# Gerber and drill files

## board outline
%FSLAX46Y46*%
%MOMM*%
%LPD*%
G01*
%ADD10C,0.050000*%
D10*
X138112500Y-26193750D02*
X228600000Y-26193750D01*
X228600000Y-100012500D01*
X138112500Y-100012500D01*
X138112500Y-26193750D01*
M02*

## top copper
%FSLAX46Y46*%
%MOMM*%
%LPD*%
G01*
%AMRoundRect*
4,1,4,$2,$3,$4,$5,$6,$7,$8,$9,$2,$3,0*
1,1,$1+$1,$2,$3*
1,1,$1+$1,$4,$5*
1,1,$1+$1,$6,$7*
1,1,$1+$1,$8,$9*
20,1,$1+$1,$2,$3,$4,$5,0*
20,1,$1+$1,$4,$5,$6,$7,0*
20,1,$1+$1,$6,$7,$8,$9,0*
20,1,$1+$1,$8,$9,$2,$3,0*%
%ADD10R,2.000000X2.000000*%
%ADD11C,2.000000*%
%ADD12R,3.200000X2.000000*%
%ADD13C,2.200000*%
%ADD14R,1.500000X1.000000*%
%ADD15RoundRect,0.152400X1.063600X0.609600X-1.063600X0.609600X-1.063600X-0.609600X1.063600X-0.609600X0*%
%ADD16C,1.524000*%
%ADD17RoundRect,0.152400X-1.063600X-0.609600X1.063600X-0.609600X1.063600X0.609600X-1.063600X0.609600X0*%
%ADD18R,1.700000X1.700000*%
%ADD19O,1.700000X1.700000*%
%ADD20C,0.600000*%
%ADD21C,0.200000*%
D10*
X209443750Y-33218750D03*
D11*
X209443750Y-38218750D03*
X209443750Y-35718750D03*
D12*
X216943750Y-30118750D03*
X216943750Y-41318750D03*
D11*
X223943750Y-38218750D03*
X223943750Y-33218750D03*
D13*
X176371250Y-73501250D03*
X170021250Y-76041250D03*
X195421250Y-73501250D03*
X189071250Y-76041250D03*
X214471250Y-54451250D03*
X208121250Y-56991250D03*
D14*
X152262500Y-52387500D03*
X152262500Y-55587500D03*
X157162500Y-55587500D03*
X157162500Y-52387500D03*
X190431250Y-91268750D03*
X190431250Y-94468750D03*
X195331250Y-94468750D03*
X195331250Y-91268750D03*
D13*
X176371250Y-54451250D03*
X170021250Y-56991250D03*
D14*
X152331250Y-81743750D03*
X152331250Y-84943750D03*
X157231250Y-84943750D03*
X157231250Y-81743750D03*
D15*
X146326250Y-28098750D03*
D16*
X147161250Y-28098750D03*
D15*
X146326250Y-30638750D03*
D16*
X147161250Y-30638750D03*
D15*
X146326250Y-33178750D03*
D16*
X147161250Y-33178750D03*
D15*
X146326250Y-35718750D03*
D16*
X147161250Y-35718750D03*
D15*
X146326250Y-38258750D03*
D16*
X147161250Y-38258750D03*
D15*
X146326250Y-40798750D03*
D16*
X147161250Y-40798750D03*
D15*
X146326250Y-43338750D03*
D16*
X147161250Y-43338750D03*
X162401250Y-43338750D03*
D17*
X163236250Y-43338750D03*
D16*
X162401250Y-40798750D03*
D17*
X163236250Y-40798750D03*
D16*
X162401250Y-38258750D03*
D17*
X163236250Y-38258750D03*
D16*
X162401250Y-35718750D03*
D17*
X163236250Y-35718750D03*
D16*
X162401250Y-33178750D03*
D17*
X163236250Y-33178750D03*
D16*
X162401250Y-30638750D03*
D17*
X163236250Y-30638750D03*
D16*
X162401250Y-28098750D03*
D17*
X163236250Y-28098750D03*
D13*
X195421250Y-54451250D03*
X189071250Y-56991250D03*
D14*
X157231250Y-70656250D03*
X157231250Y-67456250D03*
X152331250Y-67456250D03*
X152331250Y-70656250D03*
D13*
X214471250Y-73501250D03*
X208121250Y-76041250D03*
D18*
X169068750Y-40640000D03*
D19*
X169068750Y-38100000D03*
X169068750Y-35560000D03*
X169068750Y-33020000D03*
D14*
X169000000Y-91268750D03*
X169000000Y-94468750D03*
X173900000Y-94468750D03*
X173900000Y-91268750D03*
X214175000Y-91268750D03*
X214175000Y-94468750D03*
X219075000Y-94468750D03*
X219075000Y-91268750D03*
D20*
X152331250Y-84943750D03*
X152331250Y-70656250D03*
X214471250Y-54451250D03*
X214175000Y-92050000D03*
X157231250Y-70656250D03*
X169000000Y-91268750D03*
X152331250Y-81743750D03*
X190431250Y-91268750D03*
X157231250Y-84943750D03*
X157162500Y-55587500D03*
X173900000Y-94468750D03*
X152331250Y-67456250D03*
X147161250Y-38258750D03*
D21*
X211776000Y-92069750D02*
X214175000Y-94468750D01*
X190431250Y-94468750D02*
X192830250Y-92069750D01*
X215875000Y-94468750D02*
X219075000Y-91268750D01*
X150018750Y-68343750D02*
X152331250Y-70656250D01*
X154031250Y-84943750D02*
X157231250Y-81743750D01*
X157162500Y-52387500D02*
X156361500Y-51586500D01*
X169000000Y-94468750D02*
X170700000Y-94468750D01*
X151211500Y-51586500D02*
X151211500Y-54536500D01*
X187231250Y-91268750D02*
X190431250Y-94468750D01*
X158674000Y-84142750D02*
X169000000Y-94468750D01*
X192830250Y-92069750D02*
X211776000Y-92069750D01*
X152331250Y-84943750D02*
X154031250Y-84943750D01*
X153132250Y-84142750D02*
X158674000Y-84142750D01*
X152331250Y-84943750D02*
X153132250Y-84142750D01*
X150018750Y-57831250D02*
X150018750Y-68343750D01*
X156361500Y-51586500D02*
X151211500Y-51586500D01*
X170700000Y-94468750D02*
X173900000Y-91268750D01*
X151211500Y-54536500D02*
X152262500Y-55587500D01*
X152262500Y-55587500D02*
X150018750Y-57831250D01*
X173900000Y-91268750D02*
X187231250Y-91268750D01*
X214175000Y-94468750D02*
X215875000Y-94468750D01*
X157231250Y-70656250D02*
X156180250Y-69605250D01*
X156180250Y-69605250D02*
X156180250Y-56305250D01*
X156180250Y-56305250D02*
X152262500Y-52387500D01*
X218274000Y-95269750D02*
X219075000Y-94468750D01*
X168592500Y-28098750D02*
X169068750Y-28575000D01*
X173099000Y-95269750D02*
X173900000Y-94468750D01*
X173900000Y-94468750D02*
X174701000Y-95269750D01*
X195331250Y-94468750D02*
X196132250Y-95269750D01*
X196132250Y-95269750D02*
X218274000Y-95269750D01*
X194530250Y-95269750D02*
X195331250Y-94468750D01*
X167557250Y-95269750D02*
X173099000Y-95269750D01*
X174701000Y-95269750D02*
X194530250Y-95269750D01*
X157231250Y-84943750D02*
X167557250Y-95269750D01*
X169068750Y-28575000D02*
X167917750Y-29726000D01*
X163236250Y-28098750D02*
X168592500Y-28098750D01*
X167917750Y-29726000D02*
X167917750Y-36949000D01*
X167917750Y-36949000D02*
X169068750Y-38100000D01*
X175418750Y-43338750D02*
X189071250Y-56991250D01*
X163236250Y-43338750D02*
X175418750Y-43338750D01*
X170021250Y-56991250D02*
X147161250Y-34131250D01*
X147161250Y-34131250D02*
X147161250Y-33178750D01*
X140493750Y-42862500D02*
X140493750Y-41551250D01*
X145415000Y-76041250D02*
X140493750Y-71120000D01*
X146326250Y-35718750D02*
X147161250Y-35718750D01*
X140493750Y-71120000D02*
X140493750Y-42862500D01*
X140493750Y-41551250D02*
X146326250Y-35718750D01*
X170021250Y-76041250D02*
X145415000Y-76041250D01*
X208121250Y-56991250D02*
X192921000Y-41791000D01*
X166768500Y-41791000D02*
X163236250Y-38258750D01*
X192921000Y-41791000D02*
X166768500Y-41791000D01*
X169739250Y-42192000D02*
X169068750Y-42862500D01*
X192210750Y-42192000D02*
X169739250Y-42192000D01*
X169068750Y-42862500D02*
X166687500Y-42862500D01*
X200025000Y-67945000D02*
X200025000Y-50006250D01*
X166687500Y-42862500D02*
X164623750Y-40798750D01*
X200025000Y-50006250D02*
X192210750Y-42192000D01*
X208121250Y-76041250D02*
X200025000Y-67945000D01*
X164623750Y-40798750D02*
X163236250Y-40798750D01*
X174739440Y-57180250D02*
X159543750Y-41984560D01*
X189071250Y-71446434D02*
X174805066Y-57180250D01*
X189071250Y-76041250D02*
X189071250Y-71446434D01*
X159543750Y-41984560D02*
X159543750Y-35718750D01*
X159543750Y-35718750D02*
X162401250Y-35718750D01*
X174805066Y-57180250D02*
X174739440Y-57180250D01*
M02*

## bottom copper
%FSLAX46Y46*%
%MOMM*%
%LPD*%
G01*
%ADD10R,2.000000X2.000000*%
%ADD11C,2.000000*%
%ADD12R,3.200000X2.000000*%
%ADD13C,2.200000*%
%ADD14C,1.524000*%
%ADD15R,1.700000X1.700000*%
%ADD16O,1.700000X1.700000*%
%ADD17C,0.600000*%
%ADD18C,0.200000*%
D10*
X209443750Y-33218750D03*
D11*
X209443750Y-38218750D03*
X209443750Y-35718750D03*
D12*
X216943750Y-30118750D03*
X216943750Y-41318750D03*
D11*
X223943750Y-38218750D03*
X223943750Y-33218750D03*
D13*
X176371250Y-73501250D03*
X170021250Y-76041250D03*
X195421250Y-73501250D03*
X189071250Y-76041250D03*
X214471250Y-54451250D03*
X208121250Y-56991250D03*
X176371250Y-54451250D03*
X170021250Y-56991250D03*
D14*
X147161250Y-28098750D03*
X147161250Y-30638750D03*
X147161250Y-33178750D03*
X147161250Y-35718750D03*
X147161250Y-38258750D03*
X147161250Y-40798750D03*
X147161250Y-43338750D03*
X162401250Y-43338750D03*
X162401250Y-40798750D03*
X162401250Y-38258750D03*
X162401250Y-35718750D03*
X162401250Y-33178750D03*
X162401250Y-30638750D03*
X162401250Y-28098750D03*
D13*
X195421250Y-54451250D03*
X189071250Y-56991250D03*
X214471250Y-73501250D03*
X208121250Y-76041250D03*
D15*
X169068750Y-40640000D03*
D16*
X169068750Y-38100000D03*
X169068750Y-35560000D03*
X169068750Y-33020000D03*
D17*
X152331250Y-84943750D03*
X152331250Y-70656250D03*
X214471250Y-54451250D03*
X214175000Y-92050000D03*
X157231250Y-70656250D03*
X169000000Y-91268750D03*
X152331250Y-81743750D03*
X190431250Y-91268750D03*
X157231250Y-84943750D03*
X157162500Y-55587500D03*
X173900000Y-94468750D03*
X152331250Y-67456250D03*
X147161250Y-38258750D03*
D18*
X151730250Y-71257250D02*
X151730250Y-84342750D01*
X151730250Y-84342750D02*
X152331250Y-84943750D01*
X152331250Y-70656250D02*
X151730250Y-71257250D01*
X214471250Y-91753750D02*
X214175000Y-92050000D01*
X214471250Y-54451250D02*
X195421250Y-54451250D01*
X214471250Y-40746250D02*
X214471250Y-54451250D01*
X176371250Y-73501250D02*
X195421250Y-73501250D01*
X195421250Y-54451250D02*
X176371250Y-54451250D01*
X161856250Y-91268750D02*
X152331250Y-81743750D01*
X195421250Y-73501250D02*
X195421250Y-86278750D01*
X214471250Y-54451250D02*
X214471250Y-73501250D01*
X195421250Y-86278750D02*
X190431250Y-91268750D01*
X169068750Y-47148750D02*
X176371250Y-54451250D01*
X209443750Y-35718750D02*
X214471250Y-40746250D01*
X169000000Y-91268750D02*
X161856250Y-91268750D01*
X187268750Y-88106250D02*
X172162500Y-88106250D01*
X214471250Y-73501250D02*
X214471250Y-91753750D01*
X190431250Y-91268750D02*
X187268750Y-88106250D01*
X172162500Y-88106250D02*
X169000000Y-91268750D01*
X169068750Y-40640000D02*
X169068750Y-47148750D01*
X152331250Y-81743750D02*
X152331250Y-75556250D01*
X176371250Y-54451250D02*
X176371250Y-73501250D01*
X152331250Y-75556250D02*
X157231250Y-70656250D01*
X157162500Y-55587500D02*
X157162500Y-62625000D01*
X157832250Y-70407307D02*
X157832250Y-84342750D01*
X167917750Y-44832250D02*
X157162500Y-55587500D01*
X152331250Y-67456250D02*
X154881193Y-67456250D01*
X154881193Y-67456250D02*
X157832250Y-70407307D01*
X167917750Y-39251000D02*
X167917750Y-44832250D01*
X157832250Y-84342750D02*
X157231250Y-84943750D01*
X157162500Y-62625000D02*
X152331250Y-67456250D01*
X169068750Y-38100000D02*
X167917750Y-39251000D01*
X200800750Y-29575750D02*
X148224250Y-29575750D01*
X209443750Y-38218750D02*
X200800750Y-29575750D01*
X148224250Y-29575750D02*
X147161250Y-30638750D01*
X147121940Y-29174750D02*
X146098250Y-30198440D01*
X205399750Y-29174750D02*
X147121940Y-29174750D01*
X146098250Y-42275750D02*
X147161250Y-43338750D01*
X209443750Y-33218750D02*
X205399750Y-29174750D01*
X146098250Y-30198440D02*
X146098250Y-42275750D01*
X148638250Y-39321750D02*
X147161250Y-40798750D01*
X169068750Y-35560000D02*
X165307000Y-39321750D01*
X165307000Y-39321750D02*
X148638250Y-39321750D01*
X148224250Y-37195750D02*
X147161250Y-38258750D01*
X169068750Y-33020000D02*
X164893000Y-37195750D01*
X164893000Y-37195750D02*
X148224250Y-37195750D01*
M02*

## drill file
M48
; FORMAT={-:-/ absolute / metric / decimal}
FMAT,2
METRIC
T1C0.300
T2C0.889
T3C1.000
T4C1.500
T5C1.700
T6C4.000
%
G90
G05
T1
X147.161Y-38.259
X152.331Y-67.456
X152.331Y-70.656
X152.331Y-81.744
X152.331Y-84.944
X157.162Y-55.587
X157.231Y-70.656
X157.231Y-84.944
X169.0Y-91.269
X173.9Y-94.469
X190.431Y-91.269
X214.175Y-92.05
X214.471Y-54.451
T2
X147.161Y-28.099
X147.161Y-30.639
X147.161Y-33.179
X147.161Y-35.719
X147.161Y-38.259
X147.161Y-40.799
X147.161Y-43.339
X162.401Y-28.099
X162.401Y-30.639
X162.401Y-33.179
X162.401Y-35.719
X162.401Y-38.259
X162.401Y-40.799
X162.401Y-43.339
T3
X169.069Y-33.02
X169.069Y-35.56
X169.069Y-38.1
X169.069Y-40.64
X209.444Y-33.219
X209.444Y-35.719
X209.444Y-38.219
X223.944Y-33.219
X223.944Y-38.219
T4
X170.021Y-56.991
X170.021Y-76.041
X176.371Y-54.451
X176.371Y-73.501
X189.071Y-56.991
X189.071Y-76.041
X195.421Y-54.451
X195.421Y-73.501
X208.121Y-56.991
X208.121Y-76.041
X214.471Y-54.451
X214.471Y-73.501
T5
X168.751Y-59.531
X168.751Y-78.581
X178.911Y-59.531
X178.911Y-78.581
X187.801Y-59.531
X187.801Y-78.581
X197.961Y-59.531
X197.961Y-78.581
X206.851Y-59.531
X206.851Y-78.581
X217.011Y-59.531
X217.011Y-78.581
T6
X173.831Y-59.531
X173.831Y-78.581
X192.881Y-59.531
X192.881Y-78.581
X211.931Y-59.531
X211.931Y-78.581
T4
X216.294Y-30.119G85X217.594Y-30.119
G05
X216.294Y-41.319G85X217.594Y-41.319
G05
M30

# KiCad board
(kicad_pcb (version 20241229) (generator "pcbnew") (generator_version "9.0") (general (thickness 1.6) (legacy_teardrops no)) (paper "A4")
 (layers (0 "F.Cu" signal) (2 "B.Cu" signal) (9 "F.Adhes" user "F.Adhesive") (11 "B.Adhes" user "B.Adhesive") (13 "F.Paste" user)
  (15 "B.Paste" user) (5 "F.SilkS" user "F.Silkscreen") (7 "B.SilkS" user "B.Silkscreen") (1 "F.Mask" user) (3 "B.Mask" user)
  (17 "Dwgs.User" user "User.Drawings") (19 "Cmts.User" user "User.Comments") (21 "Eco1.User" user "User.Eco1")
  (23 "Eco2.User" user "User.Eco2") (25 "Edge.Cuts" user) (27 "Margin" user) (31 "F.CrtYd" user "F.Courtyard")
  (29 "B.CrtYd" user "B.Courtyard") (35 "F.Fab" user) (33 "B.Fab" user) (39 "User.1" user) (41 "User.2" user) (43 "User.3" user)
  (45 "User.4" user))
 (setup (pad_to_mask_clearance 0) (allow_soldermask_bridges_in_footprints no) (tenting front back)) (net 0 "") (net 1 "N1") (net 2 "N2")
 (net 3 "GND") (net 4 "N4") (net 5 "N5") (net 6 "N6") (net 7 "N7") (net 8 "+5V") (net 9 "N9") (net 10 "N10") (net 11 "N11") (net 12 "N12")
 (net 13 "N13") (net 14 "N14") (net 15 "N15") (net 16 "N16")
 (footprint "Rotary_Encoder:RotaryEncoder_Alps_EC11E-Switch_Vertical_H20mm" (layer "F.Cu") (at 209.44375 33.21875)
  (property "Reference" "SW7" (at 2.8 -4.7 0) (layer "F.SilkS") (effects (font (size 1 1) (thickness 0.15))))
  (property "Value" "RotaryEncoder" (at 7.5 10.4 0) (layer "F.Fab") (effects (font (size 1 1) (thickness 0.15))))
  (pad "A" thru_hole rect (at 0 0) (size 2 2) (drill 1) (layers "*.Cu" "*.Mask") (remove_unused_layers no) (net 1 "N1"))
  (pad "B" thru_hole circle (at 0 5) (size 2 2) (drill 1) (layers "*.Cu" "*.Mask") (remove_unused_layers no) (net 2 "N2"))
  (pad "C" thru_hole circle (at 0 2.5) (size 2 2) (drill 1) (layers "*.Cu" "*.Mask") (remove_unused_layers no) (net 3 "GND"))
  (pad "MP" thru_hole rect (at 7.5 -3.1) (size 3.2 2) (drill oval 2.8 1.5) (layers "*.Cu" "*.Mask") (remove_unused_layers no))
  (pad "MP" thru_hole rect (at 7.5 8.1) (size 3.2 2) (drill oval 2.8 1.5) (layers "*.Cu" "*.Mask") (remove_unused_layers no))
  (pad "S1" thru_hole circle (at 14.5 5) (size 2 2) (drill 1) (layers "*.Cu" "*.Mask") (remove_unused_layers no))
  (pad "S2" thru_hole circle (at 14.5 0) (size 2 2) (drill 1) (layers "*.Cu" "*.Mask") (remove_unused_layers no)))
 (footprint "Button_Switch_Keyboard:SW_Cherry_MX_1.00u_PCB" (layer "F.Cu") (at 176.37125 73.50125)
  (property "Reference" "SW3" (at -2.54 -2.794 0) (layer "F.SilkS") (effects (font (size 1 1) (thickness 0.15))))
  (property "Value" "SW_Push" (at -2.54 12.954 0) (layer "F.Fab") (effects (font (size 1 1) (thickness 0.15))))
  (pad "" np_thru_hole circle (at -7.62 5.08) (size 1.7 1.7) (drill 1.7) (layers "*.Cu" "*.Mask"))
  (pad "" np_thru_hole circle (at -2.54 5.08) (size 4 4) (drill 4) (layers "*.Cu" "*.Mask"))
  (pad "" np_thru_hole circle (at 2.54 5.08) (size 1.7 1.7) (drill 1.7) (layers "*.Cu" "*.Mask"))
  (pad "1" thru_hole circle (at 0 0) (size 2.2 2.2) (drill 1.5) (layers "*.Cu" "*.Mask") (remove_unused_layers no) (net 3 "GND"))
  (pad "2" thru_hole circle (at -6.35 2.54) (size 2.2 2.2) (drill 1.5) (layers "*.Cu" "*.Mask") (remove_unused_layers no) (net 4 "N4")))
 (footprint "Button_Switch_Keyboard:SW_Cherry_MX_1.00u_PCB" (layer "F.Cu") (at 195.42125 73.50125)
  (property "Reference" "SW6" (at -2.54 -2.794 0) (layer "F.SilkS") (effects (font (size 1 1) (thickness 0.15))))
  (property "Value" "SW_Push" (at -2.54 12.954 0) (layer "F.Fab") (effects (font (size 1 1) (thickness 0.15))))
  (pad "" np_thru_hole circle (at -7.62 5.08) (size 1.7 1.7) (drill 1.7) (layers "*.Cu" "*.Mask"))
  (pad "" np_thru_hole circle (at -2.54 5.08) (size 4 4) (drill 4) (layers "*.Cu" "*.Mask"))
  (pad "" np_thru_hole circle (at 2.54 5.08) (size 1.7 1.7) (drill 1.7) (layers "*.Cu" "*.Mask"))
  (pad "1" thru_hole circle (at 0 0) (size 2.2 2.2) (drill 1.5) (layers "*.Cu" "*.Mask") (remove_unused_layers no) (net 3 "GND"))
  (pad "2" thru_hole circle (at -6.35 2.54) (size 2.2 2.2) (drill 1.5) (layers "*.Cu" "*.Mask") (remove_unused_layers no) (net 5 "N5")))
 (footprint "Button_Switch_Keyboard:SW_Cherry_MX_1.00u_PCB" (layer "F.Cu") (at 214.47125 54.45125)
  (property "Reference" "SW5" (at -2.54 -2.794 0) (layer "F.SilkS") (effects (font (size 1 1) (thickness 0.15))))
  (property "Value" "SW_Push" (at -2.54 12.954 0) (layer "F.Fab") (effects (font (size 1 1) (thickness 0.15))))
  (pad "" np_thru_hole circle (at -7.62 5.08) (size 1.7 1.7) (drill 1.7) (layers "*.Cu" "*.Mask"))
  (pad "" np_thru_hole circle (at -2.54 5.08) (size 4 4) (drill 4) (layers "*.Cu" "*.Mask"))
  (pad "" np_thru_hole circle (at 2.54 5.08) (size 1.7 1.7) (drill 1.7) (layers "*.Cu" "*.Mask"))
  (pad "1" thru_hole circle (at 0 0) (size 2.2 2.2) (drill 1.5) (layers "*.Cu" "*.Mask") (remove_unused_layers no) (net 3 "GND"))
  (pad "2" thru_hole circle (at -6.35 2.54) (size 2.2 2.2) (drill 1.5) (layers "*.Cu" "*.Mask") (remove_unused_layers no) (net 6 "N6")))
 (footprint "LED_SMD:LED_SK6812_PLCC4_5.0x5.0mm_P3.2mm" (layer "F.Cu") (at 154.7125 53.9875)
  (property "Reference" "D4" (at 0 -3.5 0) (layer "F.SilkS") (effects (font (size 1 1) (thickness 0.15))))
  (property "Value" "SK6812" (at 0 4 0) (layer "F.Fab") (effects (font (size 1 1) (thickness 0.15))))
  (pad "1" smd rect (at -2.45 -1.6 180) (size 1.5 1) (layers "F.Cu" "F.Mask" "F.Paste") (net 3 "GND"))
  (pad "2" smd rect (at -2.45 1.6 180) (size 1.5 1) (layers "F.Cu" "F.Mask" "F.Paste") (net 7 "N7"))
  (pad "3" smd rect (at 2.45 1.6 180) (size 1.5 1) (layers "F.Cu" "F.Mask" "F.Paste") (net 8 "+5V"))
  (pad "4" smd rect (at 2.45 -1.6 180) (size 1.5 1) (layers "F.Cu" "F.Mask" "F.Paste") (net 7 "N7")))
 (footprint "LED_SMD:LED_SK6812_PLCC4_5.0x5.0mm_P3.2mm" (layer "F.Cu") (at 192.88125 92.86875)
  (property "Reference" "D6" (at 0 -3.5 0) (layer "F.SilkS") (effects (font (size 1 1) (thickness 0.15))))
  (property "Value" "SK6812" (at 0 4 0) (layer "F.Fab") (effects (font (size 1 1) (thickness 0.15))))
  (pad "1" smd rect (at -2.45 -1.6 180) (size 1.5 1) (layers "F.Cu" "F.Mask" "F.Paste") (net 3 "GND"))
  (pad "2" smd rect (at -2.45 1.6 180) (size 1.5 1) (layers "F.Cu" "F.Mask" "F.Paste") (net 7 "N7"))
  (pad "3" smd rect (at 2.45 1.6 180) (size 1.5 1) (layers "F.Cu" "F.Mask" "F.Paste") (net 8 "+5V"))
  (pad "4" smd rect (at 2.45 -1.6 180) (size 1.5 1) (layers "F.Cu" "F.Mask" "F.Paste") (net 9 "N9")))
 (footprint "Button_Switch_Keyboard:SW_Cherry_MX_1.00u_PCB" (layer "F.Cu") (at 176.37125 54.45125)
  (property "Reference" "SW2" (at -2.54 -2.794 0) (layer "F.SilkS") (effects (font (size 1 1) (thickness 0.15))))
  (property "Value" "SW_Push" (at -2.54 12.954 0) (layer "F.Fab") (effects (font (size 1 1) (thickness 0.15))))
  (pad "" np_thru_hole circle (at -7.62 5.08) (size 1.7 1.7) (drill 1.7) (layers "*.Cu" "*.Mask"))
  (pad "" np_thru_hole circle (at -2.54 5.08) (size 4 4) (drill 4) (layers "*.Cu" "*.Mask"))
  (pad "" np_thru_hole circle (at 2.54 5.08) (size 1.7 1.7) (drill 1.7) (layers "*.Cu" "*.Mask"))
  (pad "1" thru_hole circle (at 0 0) (size 2.2 2.2) (drill 1.5) (layers "*.Cu" "*.Mask") (remove_unused_layers no) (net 3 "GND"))
  (pad "2" thru_hole circle (at -6.35 2.54) (size 2.2 2.2) (drill 1.5) (layers "*.Cu" "*.Mask") (remove_unused_layers no) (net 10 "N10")))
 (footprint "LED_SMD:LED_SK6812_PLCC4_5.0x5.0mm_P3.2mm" (layer "F.Cu") (at 154.78125 83.34375)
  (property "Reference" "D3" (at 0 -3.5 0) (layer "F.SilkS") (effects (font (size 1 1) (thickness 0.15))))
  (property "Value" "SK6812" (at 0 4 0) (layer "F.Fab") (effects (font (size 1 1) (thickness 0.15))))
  (pad "1" smd rect (at -2.45 -1.6 180) (size 1.5 1) (layers "F.Cu" "F.Mask" "F.Paste") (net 3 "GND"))
  (pad "2" smd rect (at -2.45 1.6 180) (size 1.5 1) (layers "F.Cu" "F.Mask" "F.Paste") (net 7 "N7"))
  (pad "3" smd rect (at 2.45 1.6 180) (size 1.5 1) (layers "F.Cu" "F.Mask" "F.Paste") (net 8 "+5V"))
  (pad "4" smd rect (at 2.45 -1.6 180) (size 1.5 1) (layers "F.Cu" "F.Mask" "F.Paste") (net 7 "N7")))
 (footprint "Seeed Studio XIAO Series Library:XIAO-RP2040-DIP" (layer "F.Cu") (at 154.78125 35.71875)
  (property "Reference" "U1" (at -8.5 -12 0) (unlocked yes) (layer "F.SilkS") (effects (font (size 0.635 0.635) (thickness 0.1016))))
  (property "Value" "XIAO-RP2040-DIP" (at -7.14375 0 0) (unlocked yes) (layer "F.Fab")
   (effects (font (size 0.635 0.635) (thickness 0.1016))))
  (pad "1" smd roundrect (at -8.455 -7.62 180) (size 2.432 1.524) (layers "F.Cu" "F.Mask") (roundrect_rratio 0.1) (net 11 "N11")
   (thermal_bridge_angle 45))
  (pad "1" thru_hole circle (at -7.62 -7.62 180) (size 1.524 1.524) (drill 0.889) (layers "*.Cu" "*.Mask") (remove_unused_layers no)
   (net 11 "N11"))
  (pad "2" smd roundrect (at -8.455 -5.08 180) (size 2.432 1.524) (layers "F.Cu" "F.Mask") (roundrect_rratio 0.1) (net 2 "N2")
   (thermal_bridge_angle 45))
  (pad "2" thru_hole circle (at -7.62 -5.08 180) (size 1.524 1.524) (drill 0.889) (layers "*.Cu" "*.Mask") (remove_unused_layers no)
   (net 2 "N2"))
  (pad "3" smd roundrect (at -8.455 -2.54 180) (size 2.432 1.524) (layers "F.Cu" "F.Mask") (roundrect_rratio 0.1) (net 10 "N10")
   (thermal_bridge_angle 45))
  (pad "3" thru_hole circle (at -7.62 -2.54 180) (size 1.524 1.524) (drill 0.889) (layers "*.Cu" "*.Mask") (remove_unused_layers no)
   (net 10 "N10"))
  (pad "4" smd roundrect (at -8.455 0 180) (size 2.432 1.524) (layers "F.Cu" "F.Mask") (roundrect_rratio 0.1) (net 4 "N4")
   (thermal_bridge_angle 45))
  (pad "4" thru_hole circle (at -7.62 0 180) (size 1.524 1.524) (drill 0.889) (layers "*.Cu" "*.Mask") (remove_unused_layers no)
   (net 4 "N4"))
  (pad "5" smd roundrect (at -8.455 2.54 180) (size 2.432 1.524) (layers "F.Cu" "F.Mask") (roundrect_rratio 0.1) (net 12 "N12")
   (thermal_bridge_angle 45))
  (pad "5" thru_hole circle (at -7.62 2.54 180) (size 1.524 1.524) (drill 0.889) (layers "*.Cu" "*.Mask") (remove_unused_layers no)
   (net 12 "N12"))
  (pad "6" smd roundrect (at -8.455 5.08 180) (size 2.432 1.524) (layers "F.Cu" "F.Mask") (roundrect_rratio 0.1) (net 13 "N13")
   (thermal_bridge_angle 45))
  (pad "6" thru_hole circle (at -7.62 5.08 180) (size 1.524 1.524) (drill 0.889) (layers "*.Cu" "*.Mask") (remove_unused_layers no)
   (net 13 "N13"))
  (pad "7" smd roundrect (at -8.455 7.62 180) (size 2.432 1.524) (layers "F.Cu" "F.Mask") (roundrect_rratio 0.1) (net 1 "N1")
   (thermal_bridge_angle 45))
  (pad "7" thru_hole circle (at -7.62 7.62 180) (size 1.524 1.524) (drill 0.889) (layers "*.Cu" "*.Mask") (remove_unused_layers no)
   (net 1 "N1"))
  (pad "8" thru_hole circle (at 7.62 7.62) (size 1.524 1.524) (drill 0.889) (layers "*.Cu" "*.Mask") (remove_unused_layers no)
   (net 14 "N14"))
  (pad "8" smd roundrect (at 8.455 7.62) (size 2.432 1.524) (layers "F.Cu" "F.Mask") (roundrect_rratio 0.1) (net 14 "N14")
   (thermal_bridge_angle 45))
  (pad "9" thru_hole circle (at 7.62 5.08) (size 1.524 1.524) (drill 0.889) (layers "*.Cu" "*.Mask") (remove_unused_layers no)
   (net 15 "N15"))
  (pad "9" smd roundrect (at 8.455 5.08) (size 2.432 1.524) (layers "F.Cu" "F.Mask") (roundrect_rratio 0.1) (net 15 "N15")
   (thermal_bridge_angle 45))
  (pad "10" thru_hole circle (at 7.62 2.54) (size 1.524 1.524) (drill 0.889) (layers "*.Cu" "*.Mask") (remove_unused_layers no) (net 6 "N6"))
  (pad "10" smd roundrect (at 8.455 2.54) (size 2.432 1.524) (layers "F.Cu" "F.Mask") (roundrect_rratio 0.1) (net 6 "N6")
   (thermal_bridge_angle 45))
  (pad "11" thru_hole circle (at 7.62 0) (size 1.524 1.524) (drill 0.889) (layers "*.Cu" "*.Mask") (remove_unused_layers no) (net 5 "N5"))
  (pad "11" smd roundrect (at 8.455 0) (size 2.432 1.524) (layers "F.Cu" "F.Mask") (roundrect_rratio 0.1) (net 5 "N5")
   (thermal_bridge_angle 45))
  (pad "12" thru_hole circle (at 7.62 -2.54) (size 1.524 1.524) (drill 0.889) (layers "*.Cu" "*.Mask") (remove_unused_layers no)
   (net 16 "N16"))
  (pad "12" smd roundrect (at 8.455 -2.54) (size 2.432 1.524) (layers "F.Cu" "F.Mask") (roundrect_rratio 0.1) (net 16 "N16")
   (thermal_bridge_angle 45))
  (pad "13" thru_hole circle (at 7.62 -5.08) (size 1.524 1.524) (drill 0.889) (layers "*.Cu" "*.Mask") (remove_unused_layers no)
   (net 3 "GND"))
  (pad "13" smd roundrect (at 8.455 -5.08) (size 2.432 1.524) (layers "F.Cu" "F.Mask") (roundrect_rratio 0.1) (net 3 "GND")
   (thermal_bridge_angle 45))
  (pad "14" thru_hole circle (at 7.62 -7.62) (size 1.524 1.524) (drill 0.889) (layers "*.Cu" "*.Mask") (remove_unused_layers no)
   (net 8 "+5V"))
  (pad "14" smd roundrect (at 8.455 -7.62) (size 2.432 1.524) (layers "F.Cu" "F.Mask") (roundrect_rratio 0.1) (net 8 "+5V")
   (thermal_bridge_angle 45)))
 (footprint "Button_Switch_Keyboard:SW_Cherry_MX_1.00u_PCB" (layer "F.Cu") (at 195.42125 54.45125)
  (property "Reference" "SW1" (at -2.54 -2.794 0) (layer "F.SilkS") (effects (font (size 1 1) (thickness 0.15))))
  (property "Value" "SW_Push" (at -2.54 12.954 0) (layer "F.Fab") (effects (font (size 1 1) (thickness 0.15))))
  (pad "" np_thru_hole circle (at -7.62 5.08) (size 1.7 1.7) (drill 1.7) (layers "*.Cu" "*.Mask"))
  (pad "" np_thru_hole circle (at -2.54 5.08) (size 4 4) (drill 4) (layers "*.Cu" "*.Mask"))
  (pad "" np_thru_hole circle (at 2.54 5.08) (size 1.7 1.7) (drill 1.7) (layers "*.Cu" "*.Mask"))
  (pad "1" thru_hole circle (at 0 0) (size 2.2 2.2) (drill 1.5) (layers "*.Cu" "*.Mask") (remove_unused_layers no) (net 3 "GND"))
  (pad "2" thru_hole circle (at -6.35 2.54) (size 2.2 2.2) (drill 1.5) (layers "*.Cu" "*.Mask") (remove_unused_layers no) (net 14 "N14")))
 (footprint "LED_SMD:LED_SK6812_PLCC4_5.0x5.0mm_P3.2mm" (layer "F.Cu") (at 154.78125 69.05625 180)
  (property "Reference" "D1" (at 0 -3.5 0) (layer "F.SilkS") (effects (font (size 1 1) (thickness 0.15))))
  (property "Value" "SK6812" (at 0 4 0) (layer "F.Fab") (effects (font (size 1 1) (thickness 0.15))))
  (pad "1" smd rect (at -2.45 -1.6) (size 1.5 1) (layers "F.Cu" "F.Mask" "F.Paste") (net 3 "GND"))
  (pad "2" smd rect (at -2.45 1.6) (size 1.5 1) (layers "F.Cu" "F.Mask" "F.Paste") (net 11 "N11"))
  (pad "3" smd rect (at 2.45 1.6) (size 1.5 1) (layers "F.Cu" "F.Mask" "F.Paste") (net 8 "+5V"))
  (pad "4" smd rect (at 2.45 -1.6) (size 1.5 1) (layers "F.Cu" "F.Mask" "F.Paste") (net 7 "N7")))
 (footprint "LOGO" (layer "F.Cu") (at 145.25625 57.15)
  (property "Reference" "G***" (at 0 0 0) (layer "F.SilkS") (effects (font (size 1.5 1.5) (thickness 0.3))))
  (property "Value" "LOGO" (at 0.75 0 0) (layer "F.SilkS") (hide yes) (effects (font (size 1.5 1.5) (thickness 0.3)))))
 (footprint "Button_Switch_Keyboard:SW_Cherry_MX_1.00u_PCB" (layer "F.Cu") (at 214.47125 73.50125)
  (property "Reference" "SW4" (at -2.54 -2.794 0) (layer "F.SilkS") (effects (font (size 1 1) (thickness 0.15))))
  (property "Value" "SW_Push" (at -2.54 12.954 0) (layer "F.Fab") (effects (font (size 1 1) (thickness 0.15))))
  (pad "" np_thru_hole circle (at -7.62 5.08) (size 1.7 1.7) (drill 1.7) (layers "*.Cu" "*.Mask"))
  (pad "" np_thru_hole circle (at -2.54 5.08) (size 4 4) (drill 4) (layers "*.Cu" "*.Mask"))
  (pad "" np_thru_hole circle (at 2.54 5.08) (size 1.7 1.7) (drill 1.7) (layers "*.Cu" "*.Mask"))
  (pad "1" thru_hole circle (at 0 0) (size 2.2 2.2) (drill 1.5) (layers "*.Cu" "*.Mask") (remove_unused_layers no) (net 3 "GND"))
  (pad "2" thru_hole circle (at -6.35 2.54) (size 2.2 2.2) (drill 1.5) (layers "*.Cu" "*.Mask") (remove_unused_layers no) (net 15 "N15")))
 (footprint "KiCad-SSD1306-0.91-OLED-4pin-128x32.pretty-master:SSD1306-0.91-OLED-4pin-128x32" (layer "F.Cu") (at 205.56875 42.83 180)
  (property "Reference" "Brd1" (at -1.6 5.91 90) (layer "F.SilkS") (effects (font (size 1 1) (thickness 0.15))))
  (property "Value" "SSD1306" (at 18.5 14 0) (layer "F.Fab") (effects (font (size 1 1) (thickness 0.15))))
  (pad "1" thru_hole rect (at 36.5 2.19 180) (size 1.7 1.7) (drill 1) (layers "*.Cu" "*.Mask") (remove_unused_layers no) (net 3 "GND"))
  (pad "2" thru_hole oval (at 36.5 4.73 180) (size 1.7 1.7) (drill 1) (layers "*.Cu" "*.Mask") (remove_unused_layers no) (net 8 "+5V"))
  (pad "3" thru_hole oval (at 36.5 7.27 180) (size 1.7 1.7) (drill 1) (layers "*.Cu" "*.Mask") (remove_unused_layers no) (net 13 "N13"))
  (pad "4" thru_hole oval (at 36.5 9.81 180) (size 1.7 1.7) (drill 1) (layers "*.Cu" "*.Mask") (remove_unused_layers no) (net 12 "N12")))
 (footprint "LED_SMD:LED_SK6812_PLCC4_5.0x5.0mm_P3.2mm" (layer "F.Cu") (at 171.45 92.86875)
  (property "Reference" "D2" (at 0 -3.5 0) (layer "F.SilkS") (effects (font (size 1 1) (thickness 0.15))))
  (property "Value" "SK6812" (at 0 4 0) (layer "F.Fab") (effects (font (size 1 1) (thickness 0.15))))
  (pad "1" smd rect (at -2.45 -1.6 180) (size 1.5 1) (layers "F.Cu" "F.Mask" "F.Paste") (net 3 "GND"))
  (pad "2" smd rect (at -2.45 1.6 180) (size 1.5 1) (layers "F.Cu" "F.Mask" "F.Paste") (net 7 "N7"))
  (pad "3" smd rect (at 2.45 1.6 180) (size 1.5 1) (layers "F.Cu" "F.Mask" "F.Paste") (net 8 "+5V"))
  (pad "4" smd rect (at 2.45 -1.6 180) (size 1.5 1) (layers "F.Cu" "F.Mask" "F.Paste") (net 7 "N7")))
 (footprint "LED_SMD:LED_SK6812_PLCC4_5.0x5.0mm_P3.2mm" (layer "F.Cu") (at 216.625 92.86875)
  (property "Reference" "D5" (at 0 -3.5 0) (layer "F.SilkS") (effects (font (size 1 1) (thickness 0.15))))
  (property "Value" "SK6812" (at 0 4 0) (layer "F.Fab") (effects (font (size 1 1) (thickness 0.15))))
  (pad "1" smd rect (at -2.45 -1.6 180) (size 1.5 1) (layers "F.Cu" "F.Mask" "F.Paste") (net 3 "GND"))
  (pad "2" smd rect (at -2.45 1.6 180) (size 1.5 1) (layers "F.Cu" "F.Mask" "F.Paste") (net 7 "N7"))
  (pad "3" smd rect (at 2.45 1.6 180) (size 1.5 1) (layers "F.Cu" "F.Mask" "F.Paste") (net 8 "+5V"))
  (pad "4" smd rect (at 2.45 -1.6 180) (size 1.5 1) (layers "F.Cu" "F.Mask" "F.Paste") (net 7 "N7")))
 (gr_rect (start 138.1125 26.19375) (end 228.6 100.0125) (stroke (width 0.05) (type default)) (fill no) (layer "Edge.Cuts"))
 (segment (start 211.776 92.06975) (end 214.175 94.46875) (width 0.2) (layer "F.Cu") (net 7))
 (segment (start 190.43125 94.46875) (end 192.83025 92.06975) (width 0.2) (layer "F.Cu") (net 7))
 (segment (start 215.875 94.46875) (end 219.075 91.26875) (width 0.2) (layer "F.Cu") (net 7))
 (segment (start 150.01875 68.34375) (end 152.33125 70.65625) (width 0.2) (layer "F.Cu") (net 7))
 (segment (start 154.03125 84.94375) (end 157.23125 81.74375) (width 0.2) (layer "F.Cu") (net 7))
 (segment (start 157.1625 52.3875) (end 156.3615 51.5865) (width 0.2) (layer "F.Cu") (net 7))
 (segment (start 169 94.46875) (end 170.7 94.46875) (width 0.2) (layer "F.Cu") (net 7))
 (segment (start 151.2115 51.5865) (end 151.2115 54.5365) (width 0.2) (layer "F.Cu") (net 7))
 (segment (start 187.23125 91.26875) (end 190.43125 94.46875) (width 0.2) (layer "F.Cu") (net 7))
 (segment (start 158.674 84.14275) (end 169 94.46875) (width 0.2) (layer "F.Cu") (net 7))
 (segment (start 192.83025 92.06975) (end 211.776 92.06975) (width 0.2) (layer "F.Cu") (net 7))
 (segment (start 152.33125 84.94375) (end 154.03125 84.94375) (width 0.2) (layer "F.Cu") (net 7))
 (segment (start 153.13225 84.14275) (end 158.674 84.14275) (width 0.2) (layer "F.Cu") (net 7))
 (segment (start 152.33125 84.94375) (end 153.13225 84.14275) (width 0.2) (layer "F.Cu") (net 7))
 (segment (start 150.01875 57.83125) (end 150.01875 68.34375) (width 0.2) (layer "F.Cu") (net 7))
 (segment (start 156.3615 51.5865) (end 151.2115 51.5865) (width 0.2) (layer "F.Cu") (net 7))
 (segment (start 170.7 94.46875) (end 173.9 91.26875) (width 0.2) (layer "F.Cu") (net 7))
 (segment (start 151.2115 54.5365) (end 152.2625 55.5875) (width 0.2) (layer "F.Cu") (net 7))
 (segment (start 152.2625 55.5875) (end 150.01875 57.83125) (width 0.2) (layer "F.Cu") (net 7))
 (segment (start 173.9 91.26875) (end 187.23125 91.26875) (width 0.2) (layer "F.Cu") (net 7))
 (segment (start 214.175 94.46875) (end 215.875 94.46875) (width 0.2) (layer "F.Cu") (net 7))
 (via (at 152.33125 84.94375) (size 0.6) (drill 0.3) (layers "F.Cu" "B.Cu") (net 7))
 (via (at 152.33125 70.65625) (size 0.6) (drill 0.3) (layers "F.Cu" "B.Cu") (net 7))
 (segment (start 151.73025 71.25725) (end 151.73025 84.34275) (width 0.2) (layer "B.Cu") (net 7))
 (segment (start 151.73025 84.34275) (end 152.33125 84.94375) (width 0.2) (layer "B.Cu") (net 7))
 (segment (start 152.33125 70.65625) (end 151.73025 71.25725) (width 0.2) (layer "B.Cu") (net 7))
 (segment (start 157.23125 70.65625) (end 156.18025 69.60525) (width 0.2) (layer "F.Cu") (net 3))
 (segment (start 156.18025 69.60525) (end 156.18025 56.30525) (width 0.2) (layer "F.Cu") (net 3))
 (segment (start 156.18025 56.30525) (end 152.2625 52.3875) (width 0.2) (layer "F.Cu") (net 3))
 (via (at 214.47125 54.45125) (size 0.6) (drill 0.3) (layers "F.Cu" "B.Cu") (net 3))
 (via (at 214.175 92.05) (size 0.6) (drill 0.3) (layers "F.Cu" "B.Cu") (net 3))
 (via (at 157.23125 70.65625) (size 0.6) (drill 0.3) (layers "F.Cu" "B.Cu") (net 3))
 (via (at 169 91.26875) (size 0.6) (drill 0.3) (layers "F.Cu" "B.Cu") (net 3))
 (via (at 152.33125 81.74375) (size 0.6) (drill 0.3) (layers "F.Cu" "B.Cu") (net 3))
 (via (at 190.43125 91.26875) (size 0.6) (drill 0.3) (layers "F.Cu" "B.Cu") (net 3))
 (segment (start 214.47125 91.75375) (end 214.175 92.05) (width 0.2) (layer "B.Cu") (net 3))
 (segment (start 214.47125 54.45125) (end 195.42125 54.45125) (width 0.2) (layer "B.Cu") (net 3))
 (segment (start 214.47125 40.74625) (end 214.47125 54.45125) (width 0.2) (layer "B.Cu") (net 3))
 (segment (start 176.37125 73.50125) (end 195.42125 73.50125) (width 0.2) (layer "B.Cu") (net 3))
 (segment (start 195.42125 54.45125) (end 176.37125 54.45125) (width 0.2) (layer "B.Cu") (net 3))
 (segment (start 161.85625 91.26875) (end 152.33125 81.74375) (width 0.2) (layer "B.Cu") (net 3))
 (segment (start 195.42125 73.50125) (end 195.42125 86.27875) (width 0.2) (layer "B.Cu") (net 3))
 (segment (start 214.47125 54.45125) (end 214.47125 73.50125) (width 0.2) (layer "B.Cu") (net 3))
 (segment (start 195.42125 86.27875) (end 190.43125 91.26875) (width 0.2) (layer "B.Cu") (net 3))
 (segment (start 169.06875 47.14875) (end 176.37125 54.45125) (width 0.2) (layer "B.Cu") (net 3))
 (segment (start 209.44375 35.71875) (end 214.47125 40.74625) (width 0.2) (layer "B.Cu") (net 3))
 (segment (start 169 91.26875) (end 161.85625 91.26875) (width 0.2) (layer "B.Cu") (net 3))
 (segment (start 187.26875 88.10625) (end 172.1625 88.10625) (width 0.2) (layer "B.Cu") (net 3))
 (segment (start 214.47125 73.50125) (end 214.47125 91.75375) (width 0.2) (layer "B.Cu") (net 3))
 (segment (start 190.43125 91.26875) (end 187.26875 88.10625) (width 0.2) (layer "B.Cu") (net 3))
 (segment (start 172.1625 88.10625) (end 169 91.26875) (width 0.2) (layer "B.Cu") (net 3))
 (segment (start 169.06875 40.64) (end 169.06875 47.14875) (width 0.2) (layer "B.Cu") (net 3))
 (segment (start 152.33125 81.74375) (end 152.33125 75.55625) (width 0.2) (layer "B.Cu") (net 3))
 (segment (start 176.37125 54.45125) (end 176.37125 73.50125) (width 0.2) (layer "B.Cu") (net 3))
 (segment (start 152.33125 75.55625) (end 157.23125 70.65625) (width 0.2) (layer "B.Cu") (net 3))
 (segment (start 218.274 95.26975) (end 219.075 94.46875) (width 0.2) (layer "F.Cu") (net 8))
 (segment (start 168.5925 28.09875) (end 169.06875 28.575) (width 0.2) (layer "F.Cu") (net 8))
 (segment (start 173.099 95.26975) (end 173.9 94.46875) (width 0.2) (layer "F.Cu") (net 8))
 (segment (start 173.9 94.46875) (end 174.701 95.26975) (width 0.2) (layer "F.Cu") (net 8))
 (segment (start 195.33125 94.46875) (end 196.13225 95.26975) (width 0.2) (layer "F.Cu") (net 8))
 (segment (start 196.13225 95.26975) (end 218.274 95.26975) (width 0.2) (layer "F.Cu") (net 8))
 (segment (start 194.53025 95.26975) (end 195.33125 94.46875) (width 0.2) (layer "F.Cu") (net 8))
 (segment (start 167.55725 95.26975) (end 173.099 95.26975) (width 0.2) (layer "F.Cu") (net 8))
 (segment (start 174.701 95.26975) (end 194.53025 95.26975) (width 0.2) (layer "F.Cu") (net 8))
 (segment (start 157.23125 84.94375) (end 167.55725 95.26975) (width 0.2) (layer "F.Cu") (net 8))
 (segment (start 169.06875 28.575) (end 167.91775 29.726) (width 0.2) (layer "F.Cu") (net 8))
 (segment (start 163.23625 28.09875) (end 168.5925 28.09875) (width 0.2) (layer "F.Cu") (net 8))
 (segment (start 167.91775 29.726) (end 167.91775 36.949) (width 0.2) (layer "F.Cu") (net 8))
 (segment (start 167.91775 36.949) (end 169.06875 38.1) (width 0.2) (layer "F.Cu") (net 8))
 (via (at 157.23125 84.94375) (size 0.6) (drill 0.3) (layers "F.Cu" "B.Cu") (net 8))
 (via (at 157.1625 55.5875) (size 0.6) (drill 0.3) (layers "F.Cu" "B.Cu") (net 8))
 (via (at 173.9 94.46875) (size 0.6) (drill 0.3) (layers "F.Cu" "B.Cu") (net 8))
 (via (at 152.33125 67.45625) (size 0.6) (drill 0.3) (layers "F.Cu" "B.Cu") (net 8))
 (segment (start 157.1625 55.5875) (end 157.1625 62.625) (width 0.2) (layer "B.Cu") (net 8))
 (segment (start 157.83225 70.407307) (end 157.83225 84.34275) (width 0.2) (layer "B.Cu") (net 8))
 (segment (start 167.91775 44.83225) (end 157.1625 55.5875) (width 0.2) (layer "B.Cu") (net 8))
 (segment (start 152.33125 67.45625) (end 154.881193 67.45625) (width 0.2) (layer "B.Cu") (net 8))
 (segment (start 154.881193 67.45625) (end 157.83225 70.407307) (width 0.2) (layer "B.Cu") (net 8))
 (segment (start 167.91775 39.251) (end 167.91775 44.83225) (width 0.2) (layer "B.Cu") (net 8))
 (segment (start 157.83225 84.34275) (end 157.23125 84.94375) (width 0.2) (layer "B.Cu") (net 8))
 (segment (start 157.1625 62.625) (end 152.33125 67.45625) (width 0.2) (layer "B.Cu") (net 8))
 (segment (start 169.06875 38.1) (end 167.91775 39.251) (width 0.2) (layer "B.Cu") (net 8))
 (segment (start 175.41875 43.33875) (end 189.07125 56.99125) (width 0.2) (layer "F.Cu") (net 14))
 (segment (start 163.23625 43.33875) (end 175.41875 43.33875) (width 0.2) (layer "F.Cu") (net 14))
 (segment (start 170.02125 56.99125) (end 147.16125 34.13125) (width 0.2) (layer "F.Cu") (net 10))
 (segment (start 147.16125 34.13125) (end 147.16125 33.17875) (width 0.2) (layer "F.Cu") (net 10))
 (segment (start 140.49375 42.8625) (end 140.49375 41.55125) (width 0.2) (layer "F.Cu") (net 4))
 (segment (start 145.415 76.04125) (end 140.49375 71.12) (width 0.2) (layer "F.Cu") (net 4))
 (segment (start 146.32625 35.71875) (end 147.16125 35.71875) (width 0.2) (layer "F.Cu") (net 4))
 (segment (start 140.49375 71.12) (end 140.49375 42.8625) (width 0.2) (layer "F.Cu") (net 4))
 (segment (start 140.49375 41.55125) (end 146.32625 35.71875) (width 0.2) (layer "F.Cu") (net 4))
 (segment (start 170.02125 76.04125) (end 145.415 76.04125) (width 0.2) (layer "F.Cu") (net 4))
 (segment (start 200.80075 29.57575) (end 148.22425 29.57575) (width 0.2) (layer "B.Cu") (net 2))
 (segment (start 209.44375 38.21875) (end 200.80075 29.57575) (width 0.2) (layer "B.Cu") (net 2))
 (segment (start 148.22425 29.57575) (end 147.16125 30.63875) (width 0.2) (layer "B.Cu") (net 2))
 (segment (start 208.12125 56.99125) (end 192.921 41.791) (width 0.2) (layer "F.Cu") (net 6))
 (segment (start 166.7685 41.791) (end 163.23625 38.25875) (width 0.2) (layer "F.Cu") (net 6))
 (segment (start 192.921 41.791) (end 166.7685 41.791) (width 0.2) (layer "F.Cu") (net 6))
 (segment (start 169.73925 42.192) (end 169.06875 42.8625) (width 0.2) (layer "F.Cu") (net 15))
 (segment (start 192.21075 42.192) (end 169.73925 42.192) (width 0.2) (layer "F.Cu") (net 15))
 (segment (start 169.06875 42.8625) (end 166.6875 42.8625) (width 0.2) (layer "F.Cu") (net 15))
 (segment (start 200.025 67.945) (end 200.025 50.00625) (width 0.2) (layer "F.Cu") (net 15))
 (segment (start 166.6875 42.8625) (end 164.62375 40.79875) (width 0.2) (layer "F.Cu") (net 15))
 (segment (start 200.025 50.00625) (end 192.21075 42.192) (width 0.2) (layer "F.Cu") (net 15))
 (segment (start 208.12125 76.04125) (end 200.025 67.945) (width 0.2) (layer "F.Cu") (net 15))
 (segment (start 164.62375 40.79875) (end 163.23625 40.79875) (width 0.2) (layer "F.Cu") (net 15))
 (segment (start 147.12194 29.17475) (end 146.09825 30.19844) (width 0.2) (layer "B.Cu") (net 1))
 (segment (start 205.39975 29.17475) (end 147.12194 29.17475) (width 0.2) (layer "B.Cu") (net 1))
 (segment (start 146.09825 42.27575) (end 147.16125 43.33875) (width 0.2) (layer "B.Cu") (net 1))
 (segment (start 209.44375 33.21875) (end 205.39975 29.17475) (width 0.2) (layer "B.Cu") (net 1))
 (segment (start 146.09825 30.19844) (end 146.09825 42.27575) (width 0.2) (layer "B.Cu") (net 1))
 (segment (start 148.63825 39.32175) (end 147.16125 40.79875) (width 0.2) (layer "B.Cu") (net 13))
 (segment (start 169.06875 35.56) (end 165.307 39.32175) (width 0.2) (layer "B.Cu") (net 13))
 (segment (start 165.307 39.32175) (end 148.63825 39.32175) (width 0.2) (layer "B.Cu") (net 13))
 (via (at 147.16125 38.25875) (size 0.6) (drill 0.3) (layers "F.Cu" "B.Cu") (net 12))
 (segment (start 148.22425 37.19575) (end 147.16125 38.25875) (width 0.2) (layer "B.Cu") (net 12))
 (segment (start 169.06875 33.02) (end 164.893 37.19575) (width 0.2) (layer "B.Cu") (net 12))
 (segment (start 164.893 37.19575) (end 148.22425 37.19575) (width 0.2) (layer "B.Cu") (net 12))
 (segment (start 174.73944 57.18025) (end 159.54375 41.98456) (width 0.2) (layer "F.Cu") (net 5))
 (segment (start 189.07125 71.446434) (end 174.805066 57.18025) (width 0.2) (layer "F.Cu") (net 5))
 (segment (start 189.07125 76.04125) (end 189.07125 71.446434) (width 0.2) (layer "F.Cu") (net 5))
 (segment (start 159.54375 41.98456) (end 159.54375 35.71875) (width 0.2) (layer "F.Cu") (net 5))
 (segment (start 159.54375 35.71875) (end 162.40125 35.71875) (width 0.2) (layer "F.Cu") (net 5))
 (segment (start 174.805066 57.18025) (end 174.73944 57.18025) (width 0.2) (layer "F.Cu") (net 5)))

